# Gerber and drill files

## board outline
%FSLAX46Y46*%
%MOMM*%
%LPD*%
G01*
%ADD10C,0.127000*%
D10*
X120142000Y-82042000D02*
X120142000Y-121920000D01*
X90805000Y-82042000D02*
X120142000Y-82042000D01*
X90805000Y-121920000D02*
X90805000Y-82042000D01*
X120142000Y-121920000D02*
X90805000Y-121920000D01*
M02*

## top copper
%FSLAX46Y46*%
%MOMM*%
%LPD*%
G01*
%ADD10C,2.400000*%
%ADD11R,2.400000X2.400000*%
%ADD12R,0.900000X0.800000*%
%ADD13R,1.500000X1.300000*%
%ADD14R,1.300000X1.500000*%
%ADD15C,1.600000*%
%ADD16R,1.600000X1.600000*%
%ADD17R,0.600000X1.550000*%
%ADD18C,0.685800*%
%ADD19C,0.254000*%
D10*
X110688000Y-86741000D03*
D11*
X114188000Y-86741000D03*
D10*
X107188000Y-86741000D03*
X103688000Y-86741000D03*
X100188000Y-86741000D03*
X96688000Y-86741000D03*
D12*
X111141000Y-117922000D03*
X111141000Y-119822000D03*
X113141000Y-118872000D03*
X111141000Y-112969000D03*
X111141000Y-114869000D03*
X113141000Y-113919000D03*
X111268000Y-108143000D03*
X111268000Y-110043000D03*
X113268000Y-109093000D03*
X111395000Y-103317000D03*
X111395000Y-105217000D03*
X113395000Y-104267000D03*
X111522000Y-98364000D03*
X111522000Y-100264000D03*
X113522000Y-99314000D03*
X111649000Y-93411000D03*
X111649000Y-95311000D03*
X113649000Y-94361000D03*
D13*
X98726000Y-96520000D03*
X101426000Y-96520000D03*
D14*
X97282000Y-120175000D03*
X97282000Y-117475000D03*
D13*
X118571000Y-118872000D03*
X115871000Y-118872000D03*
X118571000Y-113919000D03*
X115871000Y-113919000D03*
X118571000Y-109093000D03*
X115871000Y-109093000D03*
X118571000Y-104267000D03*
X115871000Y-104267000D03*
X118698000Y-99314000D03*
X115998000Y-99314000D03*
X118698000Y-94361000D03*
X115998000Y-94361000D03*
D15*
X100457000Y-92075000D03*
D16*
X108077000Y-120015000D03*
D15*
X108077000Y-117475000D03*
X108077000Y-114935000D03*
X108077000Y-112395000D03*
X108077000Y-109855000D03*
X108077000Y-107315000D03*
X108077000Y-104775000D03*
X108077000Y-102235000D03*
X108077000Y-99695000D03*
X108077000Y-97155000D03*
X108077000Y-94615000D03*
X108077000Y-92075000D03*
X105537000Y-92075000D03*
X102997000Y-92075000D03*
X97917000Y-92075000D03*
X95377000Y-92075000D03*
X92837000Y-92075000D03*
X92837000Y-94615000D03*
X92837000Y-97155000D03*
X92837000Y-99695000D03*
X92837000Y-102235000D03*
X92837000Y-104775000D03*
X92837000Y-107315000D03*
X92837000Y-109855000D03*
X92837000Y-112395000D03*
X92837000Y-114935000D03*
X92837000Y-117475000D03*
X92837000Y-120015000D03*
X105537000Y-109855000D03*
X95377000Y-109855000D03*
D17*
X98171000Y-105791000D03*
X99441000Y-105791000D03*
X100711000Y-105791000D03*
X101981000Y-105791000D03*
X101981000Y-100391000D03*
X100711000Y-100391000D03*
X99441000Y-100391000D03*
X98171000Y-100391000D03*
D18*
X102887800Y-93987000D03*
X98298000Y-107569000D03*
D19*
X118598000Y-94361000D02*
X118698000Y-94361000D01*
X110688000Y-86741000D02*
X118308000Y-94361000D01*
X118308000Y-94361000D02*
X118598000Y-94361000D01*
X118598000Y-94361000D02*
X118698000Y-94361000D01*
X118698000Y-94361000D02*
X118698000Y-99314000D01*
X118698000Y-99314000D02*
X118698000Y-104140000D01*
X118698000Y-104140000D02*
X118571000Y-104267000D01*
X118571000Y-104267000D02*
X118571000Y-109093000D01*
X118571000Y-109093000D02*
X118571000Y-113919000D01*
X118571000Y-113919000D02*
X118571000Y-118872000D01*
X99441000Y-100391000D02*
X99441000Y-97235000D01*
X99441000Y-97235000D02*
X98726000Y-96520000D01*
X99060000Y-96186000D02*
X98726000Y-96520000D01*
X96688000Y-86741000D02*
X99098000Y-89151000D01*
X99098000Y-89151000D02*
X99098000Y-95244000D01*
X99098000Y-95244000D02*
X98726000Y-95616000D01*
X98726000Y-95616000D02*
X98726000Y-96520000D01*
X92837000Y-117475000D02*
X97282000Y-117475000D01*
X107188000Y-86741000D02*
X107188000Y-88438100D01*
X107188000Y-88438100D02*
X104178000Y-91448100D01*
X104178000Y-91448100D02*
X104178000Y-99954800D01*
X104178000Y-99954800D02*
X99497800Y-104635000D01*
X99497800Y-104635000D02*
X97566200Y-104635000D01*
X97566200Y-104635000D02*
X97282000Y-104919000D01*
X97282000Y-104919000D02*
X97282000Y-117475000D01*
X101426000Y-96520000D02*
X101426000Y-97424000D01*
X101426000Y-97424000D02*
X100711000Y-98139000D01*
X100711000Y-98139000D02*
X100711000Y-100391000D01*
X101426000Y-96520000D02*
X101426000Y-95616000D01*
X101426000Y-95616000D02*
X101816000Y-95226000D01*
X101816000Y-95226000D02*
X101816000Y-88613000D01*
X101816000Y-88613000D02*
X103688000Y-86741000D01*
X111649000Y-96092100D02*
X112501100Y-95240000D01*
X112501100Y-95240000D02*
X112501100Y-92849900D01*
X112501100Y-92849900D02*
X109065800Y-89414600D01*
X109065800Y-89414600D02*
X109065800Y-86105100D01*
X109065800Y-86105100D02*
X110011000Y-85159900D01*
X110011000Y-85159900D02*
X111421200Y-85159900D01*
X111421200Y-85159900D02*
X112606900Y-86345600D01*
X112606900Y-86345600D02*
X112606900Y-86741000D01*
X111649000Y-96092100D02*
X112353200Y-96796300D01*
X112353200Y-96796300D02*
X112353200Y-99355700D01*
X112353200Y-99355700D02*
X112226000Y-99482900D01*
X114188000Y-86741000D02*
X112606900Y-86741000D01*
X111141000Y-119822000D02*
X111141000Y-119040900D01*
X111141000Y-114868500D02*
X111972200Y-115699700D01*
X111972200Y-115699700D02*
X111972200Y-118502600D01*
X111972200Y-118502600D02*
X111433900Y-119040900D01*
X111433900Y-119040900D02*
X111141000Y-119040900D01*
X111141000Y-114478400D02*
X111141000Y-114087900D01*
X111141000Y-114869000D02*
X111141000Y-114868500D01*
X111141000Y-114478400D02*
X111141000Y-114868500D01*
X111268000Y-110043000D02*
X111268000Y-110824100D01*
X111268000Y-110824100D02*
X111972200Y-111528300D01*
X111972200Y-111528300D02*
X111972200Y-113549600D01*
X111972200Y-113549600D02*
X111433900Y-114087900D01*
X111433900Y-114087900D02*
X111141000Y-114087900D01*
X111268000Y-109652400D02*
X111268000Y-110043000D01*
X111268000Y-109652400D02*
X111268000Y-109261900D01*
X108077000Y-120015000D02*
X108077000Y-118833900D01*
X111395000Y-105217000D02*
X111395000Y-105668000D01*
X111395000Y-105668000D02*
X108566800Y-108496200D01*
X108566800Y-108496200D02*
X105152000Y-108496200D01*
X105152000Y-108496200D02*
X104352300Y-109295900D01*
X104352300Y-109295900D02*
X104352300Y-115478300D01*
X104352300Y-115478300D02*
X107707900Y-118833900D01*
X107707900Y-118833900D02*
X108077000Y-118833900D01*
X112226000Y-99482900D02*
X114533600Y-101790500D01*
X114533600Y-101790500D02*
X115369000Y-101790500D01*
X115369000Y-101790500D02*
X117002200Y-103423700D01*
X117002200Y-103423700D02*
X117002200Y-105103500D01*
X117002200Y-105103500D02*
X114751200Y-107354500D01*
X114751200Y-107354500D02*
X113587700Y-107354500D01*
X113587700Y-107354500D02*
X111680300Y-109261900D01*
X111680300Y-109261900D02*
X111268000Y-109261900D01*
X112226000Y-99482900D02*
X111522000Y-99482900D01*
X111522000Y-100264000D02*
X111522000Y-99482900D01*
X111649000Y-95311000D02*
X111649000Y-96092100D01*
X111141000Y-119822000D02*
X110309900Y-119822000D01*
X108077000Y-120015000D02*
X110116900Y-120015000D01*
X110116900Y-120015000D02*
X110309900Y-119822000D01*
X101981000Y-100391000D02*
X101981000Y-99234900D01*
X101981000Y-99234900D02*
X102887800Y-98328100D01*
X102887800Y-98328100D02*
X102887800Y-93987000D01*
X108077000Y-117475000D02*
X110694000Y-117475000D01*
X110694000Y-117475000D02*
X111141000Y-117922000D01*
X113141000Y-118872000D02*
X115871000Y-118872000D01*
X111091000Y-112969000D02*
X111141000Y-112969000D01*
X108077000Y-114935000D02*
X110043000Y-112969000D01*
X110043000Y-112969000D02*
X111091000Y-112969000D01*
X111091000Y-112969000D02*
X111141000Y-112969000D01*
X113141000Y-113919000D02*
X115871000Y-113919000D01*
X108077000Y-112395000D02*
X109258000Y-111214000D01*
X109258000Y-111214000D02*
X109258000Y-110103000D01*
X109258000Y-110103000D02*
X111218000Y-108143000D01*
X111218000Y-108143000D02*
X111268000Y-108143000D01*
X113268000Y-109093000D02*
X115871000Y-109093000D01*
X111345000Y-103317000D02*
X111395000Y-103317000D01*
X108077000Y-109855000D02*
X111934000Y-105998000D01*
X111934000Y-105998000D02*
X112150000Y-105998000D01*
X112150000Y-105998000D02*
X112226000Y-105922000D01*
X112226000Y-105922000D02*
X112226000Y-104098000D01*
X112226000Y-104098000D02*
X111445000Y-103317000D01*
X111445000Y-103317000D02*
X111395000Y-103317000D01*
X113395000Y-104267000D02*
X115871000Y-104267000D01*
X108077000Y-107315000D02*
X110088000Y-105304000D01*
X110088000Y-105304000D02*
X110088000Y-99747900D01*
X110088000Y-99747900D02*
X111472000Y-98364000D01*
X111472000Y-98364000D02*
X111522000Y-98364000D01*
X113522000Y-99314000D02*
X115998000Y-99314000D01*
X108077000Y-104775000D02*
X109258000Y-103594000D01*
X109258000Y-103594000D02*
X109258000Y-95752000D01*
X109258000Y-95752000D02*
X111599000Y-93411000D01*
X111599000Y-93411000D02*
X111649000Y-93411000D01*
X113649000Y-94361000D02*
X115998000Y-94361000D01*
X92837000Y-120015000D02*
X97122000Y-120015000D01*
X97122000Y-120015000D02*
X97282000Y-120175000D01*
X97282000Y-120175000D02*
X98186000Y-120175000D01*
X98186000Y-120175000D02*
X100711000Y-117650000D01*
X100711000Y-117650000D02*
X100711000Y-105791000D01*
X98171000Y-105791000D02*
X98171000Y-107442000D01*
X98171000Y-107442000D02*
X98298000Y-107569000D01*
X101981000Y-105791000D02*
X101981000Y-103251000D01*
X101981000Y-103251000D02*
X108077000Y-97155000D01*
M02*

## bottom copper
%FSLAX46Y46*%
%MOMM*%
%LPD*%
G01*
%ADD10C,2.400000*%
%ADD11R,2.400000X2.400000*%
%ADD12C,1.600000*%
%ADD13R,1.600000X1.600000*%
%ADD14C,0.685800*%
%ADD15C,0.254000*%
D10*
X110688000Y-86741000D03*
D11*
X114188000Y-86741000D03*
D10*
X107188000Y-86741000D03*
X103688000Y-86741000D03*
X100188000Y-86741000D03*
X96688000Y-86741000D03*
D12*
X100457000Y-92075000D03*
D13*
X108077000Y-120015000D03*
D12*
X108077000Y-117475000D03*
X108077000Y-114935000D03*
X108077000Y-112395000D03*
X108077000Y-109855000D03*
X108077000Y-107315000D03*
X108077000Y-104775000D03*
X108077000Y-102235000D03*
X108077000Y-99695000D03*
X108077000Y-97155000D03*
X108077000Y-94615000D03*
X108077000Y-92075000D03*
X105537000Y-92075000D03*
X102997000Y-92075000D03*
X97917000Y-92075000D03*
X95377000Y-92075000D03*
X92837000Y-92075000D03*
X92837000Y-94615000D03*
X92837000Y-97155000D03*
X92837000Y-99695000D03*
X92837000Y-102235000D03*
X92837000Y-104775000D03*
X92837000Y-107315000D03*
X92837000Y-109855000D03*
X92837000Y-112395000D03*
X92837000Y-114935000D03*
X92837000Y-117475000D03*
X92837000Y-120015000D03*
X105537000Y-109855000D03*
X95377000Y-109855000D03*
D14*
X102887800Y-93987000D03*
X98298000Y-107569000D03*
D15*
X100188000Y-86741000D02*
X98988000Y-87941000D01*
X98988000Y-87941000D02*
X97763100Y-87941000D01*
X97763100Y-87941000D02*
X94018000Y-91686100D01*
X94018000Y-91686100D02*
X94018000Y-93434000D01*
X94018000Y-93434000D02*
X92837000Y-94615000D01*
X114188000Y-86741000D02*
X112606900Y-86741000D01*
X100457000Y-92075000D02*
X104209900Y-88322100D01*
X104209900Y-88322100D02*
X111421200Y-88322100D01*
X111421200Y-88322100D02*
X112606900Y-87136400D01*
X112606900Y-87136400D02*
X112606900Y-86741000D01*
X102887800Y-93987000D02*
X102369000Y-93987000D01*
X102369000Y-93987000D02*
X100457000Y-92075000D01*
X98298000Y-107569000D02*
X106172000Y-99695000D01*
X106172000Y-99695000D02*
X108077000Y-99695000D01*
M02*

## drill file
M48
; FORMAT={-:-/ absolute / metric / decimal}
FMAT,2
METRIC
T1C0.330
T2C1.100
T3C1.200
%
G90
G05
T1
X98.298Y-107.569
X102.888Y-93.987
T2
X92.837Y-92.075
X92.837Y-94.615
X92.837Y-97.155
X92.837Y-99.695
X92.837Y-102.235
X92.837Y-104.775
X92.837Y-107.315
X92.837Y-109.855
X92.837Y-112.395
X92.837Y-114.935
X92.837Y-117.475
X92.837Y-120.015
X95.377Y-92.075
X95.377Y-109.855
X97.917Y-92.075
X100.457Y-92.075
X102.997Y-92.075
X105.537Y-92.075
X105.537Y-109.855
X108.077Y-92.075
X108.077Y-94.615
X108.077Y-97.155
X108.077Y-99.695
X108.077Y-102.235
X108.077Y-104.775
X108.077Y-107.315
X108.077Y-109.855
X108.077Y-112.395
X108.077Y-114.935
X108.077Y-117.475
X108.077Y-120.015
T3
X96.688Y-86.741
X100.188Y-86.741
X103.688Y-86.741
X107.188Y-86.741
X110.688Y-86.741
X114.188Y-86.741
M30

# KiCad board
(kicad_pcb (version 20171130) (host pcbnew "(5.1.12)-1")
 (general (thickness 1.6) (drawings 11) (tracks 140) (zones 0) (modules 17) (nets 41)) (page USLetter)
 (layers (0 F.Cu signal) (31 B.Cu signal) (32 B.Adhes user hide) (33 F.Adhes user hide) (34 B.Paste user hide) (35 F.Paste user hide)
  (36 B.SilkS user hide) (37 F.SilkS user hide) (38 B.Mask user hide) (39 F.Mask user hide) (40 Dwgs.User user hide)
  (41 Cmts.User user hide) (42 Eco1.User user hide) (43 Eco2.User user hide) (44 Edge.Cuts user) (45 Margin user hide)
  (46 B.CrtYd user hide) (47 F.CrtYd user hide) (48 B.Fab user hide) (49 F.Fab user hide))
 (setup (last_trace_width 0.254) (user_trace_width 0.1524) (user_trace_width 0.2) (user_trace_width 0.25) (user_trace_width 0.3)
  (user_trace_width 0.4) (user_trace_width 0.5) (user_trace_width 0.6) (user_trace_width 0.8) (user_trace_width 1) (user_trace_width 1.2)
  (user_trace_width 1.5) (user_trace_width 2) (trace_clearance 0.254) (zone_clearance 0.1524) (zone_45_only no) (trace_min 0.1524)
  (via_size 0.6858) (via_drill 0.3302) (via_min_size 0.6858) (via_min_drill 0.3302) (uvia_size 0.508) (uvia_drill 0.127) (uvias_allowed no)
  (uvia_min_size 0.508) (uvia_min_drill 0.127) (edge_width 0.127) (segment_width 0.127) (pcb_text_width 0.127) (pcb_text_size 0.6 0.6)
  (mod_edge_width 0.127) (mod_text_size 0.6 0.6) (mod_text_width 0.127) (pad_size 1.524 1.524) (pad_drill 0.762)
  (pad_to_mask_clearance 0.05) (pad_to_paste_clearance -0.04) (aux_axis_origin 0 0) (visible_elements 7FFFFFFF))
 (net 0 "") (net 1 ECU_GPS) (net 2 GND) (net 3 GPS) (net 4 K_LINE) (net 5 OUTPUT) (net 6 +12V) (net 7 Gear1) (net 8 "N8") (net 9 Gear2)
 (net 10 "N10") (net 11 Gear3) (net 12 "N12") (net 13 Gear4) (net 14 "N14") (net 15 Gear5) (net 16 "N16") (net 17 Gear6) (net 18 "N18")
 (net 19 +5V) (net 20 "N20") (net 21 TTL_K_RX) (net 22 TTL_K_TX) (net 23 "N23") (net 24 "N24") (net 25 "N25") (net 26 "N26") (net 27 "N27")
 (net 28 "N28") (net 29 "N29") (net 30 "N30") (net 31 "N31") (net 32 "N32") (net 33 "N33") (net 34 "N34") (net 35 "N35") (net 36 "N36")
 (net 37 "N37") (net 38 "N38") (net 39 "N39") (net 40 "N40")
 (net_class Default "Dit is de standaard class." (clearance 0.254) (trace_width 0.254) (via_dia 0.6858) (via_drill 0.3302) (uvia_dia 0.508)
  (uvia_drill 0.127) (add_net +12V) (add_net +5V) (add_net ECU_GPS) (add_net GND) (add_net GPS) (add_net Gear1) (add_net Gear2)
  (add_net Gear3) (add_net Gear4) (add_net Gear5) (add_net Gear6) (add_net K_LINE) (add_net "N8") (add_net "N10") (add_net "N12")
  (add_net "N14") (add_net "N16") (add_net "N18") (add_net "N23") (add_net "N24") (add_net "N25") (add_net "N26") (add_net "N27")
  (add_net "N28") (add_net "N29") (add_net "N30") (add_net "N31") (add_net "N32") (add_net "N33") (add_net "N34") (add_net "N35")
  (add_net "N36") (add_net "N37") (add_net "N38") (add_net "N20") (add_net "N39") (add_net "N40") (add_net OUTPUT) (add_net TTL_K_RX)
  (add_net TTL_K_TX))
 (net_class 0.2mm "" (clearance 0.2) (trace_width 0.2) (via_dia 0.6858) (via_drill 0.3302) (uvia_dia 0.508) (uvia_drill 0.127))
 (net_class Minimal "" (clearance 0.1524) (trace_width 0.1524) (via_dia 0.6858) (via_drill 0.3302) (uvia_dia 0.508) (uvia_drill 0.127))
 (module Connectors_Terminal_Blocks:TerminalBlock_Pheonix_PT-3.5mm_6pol (layer F.Cu) (at 114.188 86.741 180)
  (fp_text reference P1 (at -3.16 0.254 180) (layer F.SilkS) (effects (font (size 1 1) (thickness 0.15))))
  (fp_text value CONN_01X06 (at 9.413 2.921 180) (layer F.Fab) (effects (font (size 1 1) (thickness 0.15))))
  (pad 2 thru_hole circle (at 3.5 0 180) (size 2.4 2.4) (drill 1.2) (layers *.Cu *.Mask) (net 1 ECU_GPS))
  (pad 1 thru_hole rect (at 0 0 180) (size 2.4 2.4) (drill 1.2) (layers *.Cu *.Mask) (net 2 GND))
  (pad 3 thru_hole circle (at 7 0 180) (size 2.4 2.4) (drill 1.2) (layers *.Cu *.Mask) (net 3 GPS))
  (pad 4 thru_hole circle (at 10.5 0 180) (size 2.4 2.4) (drill 1.2) (layers *.Cu *.Mask) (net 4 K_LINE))
  (pad 5 thru_hole circle (at 14 0 180) (size 2.4 2.4) (drill 1.2) (layers *.Cu *.Mask) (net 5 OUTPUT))
  (pad 6 thru_hole circle (at 17.5 0 180) (size 2.4 2.4) (drill 1.2) (layers *.Cu *.Mask) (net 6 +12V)))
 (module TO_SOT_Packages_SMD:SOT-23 (layer F.Cu) (at 112.141 118.872)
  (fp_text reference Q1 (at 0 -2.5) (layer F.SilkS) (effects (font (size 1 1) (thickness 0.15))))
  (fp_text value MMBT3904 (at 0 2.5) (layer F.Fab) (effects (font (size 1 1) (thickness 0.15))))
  (pad 1 smd rect (at -1 -0.95) (size 0.9 0.8) (layers F.Cu F.Paste F.Mask) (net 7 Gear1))
  (pad 2 smd rect (at -1 0.95) (size 0.9 0.8) (layers F.Cu F.Paste F.Mask) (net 2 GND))
  (pad 3 smd rect (at 1 0) (size 0.9 0.8) (layers F.Cu F.Paste F.Mask) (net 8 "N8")))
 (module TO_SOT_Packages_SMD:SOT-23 (layer F.Cu) (at 112.141 113.919)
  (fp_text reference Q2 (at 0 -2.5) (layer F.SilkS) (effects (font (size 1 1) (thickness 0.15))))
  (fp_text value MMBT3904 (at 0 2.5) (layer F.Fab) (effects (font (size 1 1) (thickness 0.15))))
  (pad 1 smd rect (at -1 -0.95) (size 0.9 0.8) (layers F.Cu F.Paste F.Mask) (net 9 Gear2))
  (pad 2 smd rect (at -1 0.95) (size 0.9 0.8) (layers F.Cu F.Paste F.Mask) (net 2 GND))
  (pad 3 smd rect (at 1 0) (size 0.9 0.8) (layers F.Cu F.Paste F.Mask) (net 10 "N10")))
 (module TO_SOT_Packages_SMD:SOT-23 (layer F.Cu) (at 112.268 109.093)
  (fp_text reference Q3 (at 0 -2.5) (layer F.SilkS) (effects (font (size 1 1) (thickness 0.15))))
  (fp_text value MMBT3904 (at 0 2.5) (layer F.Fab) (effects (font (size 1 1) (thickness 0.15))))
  (pad 1 smd rect (at -1 -0.95) (size 0.9 0.8) (layers F.Cu F.Paste F.Mask) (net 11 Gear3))
  (pad 2 smd rect (at -1 0.95) (size 0.9 0.8) (layers F.Cu F.Paste F.Mask) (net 2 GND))
  (pad 3 smd rect (at 1 0) (size 0.9 0.8) (layers F.Cu F.Paste F.Mask) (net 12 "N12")))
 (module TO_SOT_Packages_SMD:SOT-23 (layer F.Cu) (at 112.395 104.267)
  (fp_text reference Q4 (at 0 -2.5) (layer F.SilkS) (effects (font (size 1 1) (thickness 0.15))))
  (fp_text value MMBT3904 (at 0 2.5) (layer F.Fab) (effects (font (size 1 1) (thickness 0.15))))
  (pad 1 smd rect (at -1 -0.95) (size 0.9 0.8) (layers F.Cu F.Paste F.Mask) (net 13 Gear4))
  (pad 2 smd rect (at -1 0.95) (size 0.9 0.8) (layers F.Cu F.Paste F.Mask) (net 2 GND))
  (pad 3 smd rect (at 1 0) (size 0.9 0.8) (layers F.Cu F.Paste F.Mask) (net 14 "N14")))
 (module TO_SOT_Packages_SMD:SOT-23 (layer F.Cu) (at 112.522 99.314)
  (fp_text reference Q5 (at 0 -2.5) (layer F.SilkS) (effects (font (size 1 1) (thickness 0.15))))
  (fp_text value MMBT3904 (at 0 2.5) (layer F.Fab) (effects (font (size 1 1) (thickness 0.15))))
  (pad 1 smd rect (at -1 -0.95) (size 0.9 0.8) (layers F.Cu F.Paste F.Mask) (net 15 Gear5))
  (pad 2 smd rect (at -1 0.95) (size 0.9 0.8) (layers F.Cu F.Paste F.Mask) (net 2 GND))
  (pad 3 smd rect (at 1 0) (size 0.9 0.8) (layers F.Cu F.Paste F.Mask) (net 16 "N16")))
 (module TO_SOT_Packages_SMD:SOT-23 (layer F.Cu) (at 112.649 94.361)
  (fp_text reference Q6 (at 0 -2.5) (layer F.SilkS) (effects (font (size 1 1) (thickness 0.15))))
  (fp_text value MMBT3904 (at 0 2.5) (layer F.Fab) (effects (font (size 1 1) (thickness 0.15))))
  (pad 1 smd rect (at -1 -0.95) (size 0.9 0.8) (layers F.Cu F.Paste F.Mask) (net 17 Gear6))
  (pad 2 smd rect (at -1 0.95) (size 0.9 0.8) (layers F.Cu F.Paste F.Mask) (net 2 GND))
  (pad 3 smd rect (at 1 0) (size 0.9 0.8) (layers F.Cu F.Paste F.Mask) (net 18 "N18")))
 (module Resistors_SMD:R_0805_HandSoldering (layer F.Cu) (at 100.076 96.52)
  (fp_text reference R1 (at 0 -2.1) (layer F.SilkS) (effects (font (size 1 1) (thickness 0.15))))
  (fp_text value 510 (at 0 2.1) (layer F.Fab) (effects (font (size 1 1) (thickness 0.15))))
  (pad 1 smd rect (at -1.35 0) (size 1.5 1.3) (layers F.Cu F.Paste F.Mask) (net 6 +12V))
  (pad 2 smd rect (at 1.35 0) (size 1.5 1.3) (layers F.Cu F.Paste F.Mask) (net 4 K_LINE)))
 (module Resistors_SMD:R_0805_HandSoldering (layer F.Cu) (at 97.282 118.825 90)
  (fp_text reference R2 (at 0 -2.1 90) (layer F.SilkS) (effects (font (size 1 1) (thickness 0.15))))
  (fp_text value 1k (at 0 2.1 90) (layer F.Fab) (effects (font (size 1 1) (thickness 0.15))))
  (pad 1 smd rect (at -1.35 0 90) (size 1.5 1.3) (layers F.Cu F.Paste F.Mask) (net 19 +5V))
  (pad 2 smd rect (at 1.35 0 90) (size 1.5 1.3) (layers F.Cu F.Paste F.Mask) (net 3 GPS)))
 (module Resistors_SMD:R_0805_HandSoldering (layer F.Cu) (at 117.221 118.872 180)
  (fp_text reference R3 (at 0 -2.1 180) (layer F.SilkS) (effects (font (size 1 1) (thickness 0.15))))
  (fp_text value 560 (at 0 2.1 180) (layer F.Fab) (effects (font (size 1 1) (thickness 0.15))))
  (pad 1 smd rect (at -1.35 0 180) (size 1.5 1.3) (layers F.Cu F.Paste F.Mask) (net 1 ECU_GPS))
  (pad 2 smd rect (at 1.35 0 180) (size 1.5 1.3) (layers F.Cu F.Paste F.Mask) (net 8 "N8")))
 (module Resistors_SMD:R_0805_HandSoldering (layer F.Cu) (at 117.221 113.919 180)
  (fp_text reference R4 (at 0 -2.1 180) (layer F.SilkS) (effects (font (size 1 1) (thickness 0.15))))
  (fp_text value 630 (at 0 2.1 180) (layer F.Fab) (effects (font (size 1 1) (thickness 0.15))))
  (pad 1 smd rect (at -1.35 0 180) (size 1.5 1.3) (layers F.Cu F.Paste F.Mask) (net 1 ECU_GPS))
  (pad 2 smd rect (at 1.35 0 180) (size 1.5 1.3) (layers F.Cu F.Paste F.Mask) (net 10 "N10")))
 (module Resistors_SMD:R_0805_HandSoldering (layer F.Cu) (at 117.221 109.093 180)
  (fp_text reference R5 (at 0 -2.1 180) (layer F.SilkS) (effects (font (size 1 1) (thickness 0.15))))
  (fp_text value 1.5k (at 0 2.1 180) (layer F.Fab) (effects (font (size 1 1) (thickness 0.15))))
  (pad 1 smd rect (at -1.35 0 180) (size 1.5 1.3) (layers F.Cu F.Paste F.Mask) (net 1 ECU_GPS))
  (pad 2 smd rect (at 1.35 0 180) (size 1.5 1.3) (layers F.Cu F.Paste F.Mask) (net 12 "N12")))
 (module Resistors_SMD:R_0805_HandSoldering (layer F.Cu) (at 117.221 104.267 180)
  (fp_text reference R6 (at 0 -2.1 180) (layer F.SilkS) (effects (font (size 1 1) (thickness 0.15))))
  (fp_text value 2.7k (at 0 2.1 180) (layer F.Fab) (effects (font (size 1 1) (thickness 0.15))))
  (pad 1 smd rect (at -1.35 0 180) (size 1.5 1.3) (layers F.Cu F.Paste F.Mask) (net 1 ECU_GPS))
  (pad 2 smd rect (at 1.35 0 180) (size 1.5 1.3) (layers F.Cu F.Paste F.Mask) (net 14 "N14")))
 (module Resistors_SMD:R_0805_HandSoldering (layer F.Cu) (at 117.348 99.314 180)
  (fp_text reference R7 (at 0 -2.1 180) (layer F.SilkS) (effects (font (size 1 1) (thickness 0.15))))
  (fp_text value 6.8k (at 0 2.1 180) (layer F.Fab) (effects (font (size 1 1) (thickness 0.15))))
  (pad 1 smd rect (at -1.35 0 180) (size 1.5 1.3) (layers F.Cu F.Paste F.Mask) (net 1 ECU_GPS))
  (pad 2 smd rect (at 1.35 0 180) (size 1.5 1.3) (layers F.Cu F.Paste F.Mask) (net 16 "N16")))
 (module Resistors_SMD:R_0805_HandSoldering (layer F.Cu) (at 117.348 94.361 180)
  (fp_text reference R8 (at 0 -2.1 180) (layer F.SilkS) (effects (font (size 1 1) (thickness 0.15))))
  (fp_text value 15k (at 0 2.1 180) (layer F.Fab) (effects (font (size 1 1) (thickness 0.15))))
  (pad 1 smd rect (at -1.35 0 180) (size 1.5 1.3) (layers F.Cu F.Paste F.Mask) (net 1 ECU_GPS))
  (pad 2 smd rect (at 1.35 0 180) (size 1.5 1.3) (layers F.Cu F.Paste F.Mask) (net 18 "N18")))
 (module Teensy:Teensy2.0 (layer F.Cu) (at 100.457 106.045 90)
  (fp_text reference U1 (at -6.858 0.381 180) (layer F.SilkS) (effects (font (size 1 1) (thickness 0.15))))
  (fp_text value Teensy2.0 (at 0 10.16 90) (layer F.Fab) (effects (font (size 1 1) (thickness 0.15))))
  (pad 15 thru_hole circle (at 13.97 0 90) (size 1.6 1.6) (drill 1.1) (layers *.Cu *.Mask F.SilkS) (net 2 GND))
  (pad 1 thru_hole rect (at -13.97 7.62 90) (size 1.6 1.6) (drill 1.1) (layers *.Cu *.Mask F.SilkS) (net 2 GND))
  (pad 2 thru_hole circle (at -11.43 7.62 90) (size 1.6 1.6) (drill 1.1) (layers *.Cu *.Mask F.SilkS) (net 7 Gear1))
  (pad 3 thru_hole circle (at -8.89 7.62 90) (size 1.6 1.6) (drill 1.1) (layers *.Cu *.Mask F.SilkS) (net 9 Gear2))
  (pad 4 thru_hole circle (at -6.35 7.62 90) (size 1.6 1.6) (drill 1.1) (layers *.Cu *.Mask F.SilkS) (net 11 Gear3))
  (pad 5 thru_hole circle (at -3.81 7.62 90) (size 1.6 1.6) (drill 1.1) (layers *.Cu *.Mask F.SilkS) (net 13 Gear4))
  (pad 6 thru_hole circle (at -1.27 7.62 90) (size 1.6 1.6) (drill 1.1) (layers *.Cu *.Mask F.SilkS) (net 15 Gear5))
  (pad 7 thru_hole circle (at 1.27 7.62 90) (size 1.6 1.6) (drill 1.1) (layers *.Cu *.Mask F.SilkS) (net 17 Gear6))
  (pad 8 thru_hole circle (at 3.81 7.62 90) (size 1.6 1.6) (drill 1.1) (layers *.Cu *.Mask F.SilkS) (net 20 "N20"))
  (pad 9 thru_hole circle (at 6.35 7.62 90) (size 1.6 1.6) (drill 1.1) (layers *.Cu *.Mask F.SilkS) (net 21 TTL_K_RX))
  (pad 10 thru_hole circle (at 8.89 7.62 90) (size 1.6 1.6) (drill 1.1) (layers *.Cu *.Mask F.SilkS) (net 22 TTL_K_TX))
  (pad 11 thru_hole circle (at 11.43 7.62 90) (size 1.6 1.6) (drill 1.1) (layers *.Cu *.Mask F.SilkS) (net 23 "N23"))
  (pad 12 thru_hole circle (at 13.97 7.62 90) (size 1.6 1.6) (drill 1.1) (layers *.Cu *.Mask F.SilkS) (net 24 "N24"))
  (pad 13 thru_hole circle (at 13.97 5.08 90) (size 1.6 1.6) (drill 1.1) (layers *.Cu *.Mask F.SilkS) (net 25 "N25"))
  (pad 14 thru_hole circle (at 13.97 2.54 90) (size 1.6 1.6) (drill 1.1) (layers *.Cu *.Mask F.SilkS) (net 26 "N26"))
  (pad 16 thru_hole circle (at 13.97 -2.54 90) (size 1.6 1.6) (drill 1.1) (layers *.Cu *.Mask F.SilkS) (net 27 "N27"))
  (pad 17 thru_hole circle (at 13.97 -5.08 90) (size 1.6 1.6) (drill 1.1) (layers *.Cu *.Mask F.SilkS) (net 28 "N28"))
  (pad 18 thru_hole circle (at 13.97 -7.62 90) (size 1.6 1.6) (drill 1.1) (layers *.Cu *.Mask F.SilkS) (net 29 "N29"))
  (pad 19 thru_hole circle (at 11.43 -7.62 90) (size 1.6 1.6) (drill 1.1) (layers *.Cu *.Mask F.SilkS) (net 5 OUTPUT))
  (pad 20 thru_hole circle (at 8.89 -7.62 90) (size 1.6 1.6) (drill 1.1) (layers *.Cu *.Mask F.SilkS) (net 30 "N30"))
  (pad 21 thru_hole circle (at 6.35 -7.62 90) (size 1.6 1.6) (drill 1.1) (layers *.Cu *.Mask F.SilkS) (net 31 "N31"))
  (pad 22 thru_hole circle (at 3.81 -7.62 90) (size 1.6 1.6) (drill 1.1) (layers *.Cu *.Mask F.SilkS) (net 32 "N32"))
  (pad 23 thru_hole circle (at 1.27 -7.62 90) (size 1.6 1.6) (drill 1.1) (layers *.Cu *.Mask F.SilkS) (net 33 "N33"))
  (pad 24 thru_hole circle (at -1.27 -7.62 90) (size 1.6 1.6) (drill 1.1) (layers *.Cu *.Mask F.SilkS) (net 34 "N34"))
  (pad 25 thru_hole circle (at -3.81 -7.62 90) (size 1.6 1.6) (drill 1.1) (layers *.Cu *.Mask F.SilkS) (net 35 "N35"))
  (pad 26 thru_hole circle (at -6.35 -7.62 90) (size 1.6 1.6) (drill 1.1) (layers *.Cu *.Mask F.SilkS))
  (pad 27 thru_hole circle (at -8.89 -7.62 90) (size 1.6 1.6) (drill 1.1) (layers *.Cu *.Mask F.SilkS) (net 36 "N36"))
  (pad 28 thru_hole circle (at -11.43 -7.62 90) (size 1.6 1.6) (drill 1.1) (layers *.Cu *.Mask F.SilkS) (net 3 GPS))
  (pad 29 thru_hole circle (at -13.97 -7.62 90) (size 1.6 1.6) (drill 1.1) (layers *.Cu *.Mask F.SilkS) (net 19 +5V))
  (pad 30 thru_hole circle (at -3.81 5.08 90) (size 1.6 1.6) (drill 1.1) (layers *.Cu *.Mask F.SilkS) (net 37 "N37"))
  (pad 31 thru_hole circle (at -3.81 -5.08 90) (size 1.6 1.6) (drill 1.1) (layers *.Cu *.Mask F.SilkS) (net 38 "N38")))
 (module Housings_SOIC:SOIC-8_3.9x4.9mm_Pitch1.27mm (layer F.Cu) (at 100.076 103.091 90)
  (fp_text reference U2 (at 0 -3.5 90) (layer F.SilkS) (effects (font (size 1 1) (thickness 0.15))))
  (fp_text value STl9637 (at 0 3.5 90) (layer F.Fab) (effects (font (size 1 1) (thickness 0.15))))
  (pad 1 smd rect (at -2.7 -1.905 90) (size 1.55 0.6) (layers F.Cu F.Paste F.Mask) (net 21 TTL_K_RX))
  (pad 2 smd rect (at -2.7 -0.635 90) (size 1.55 0.6) (layers F.Cu F.Paste F.Mask) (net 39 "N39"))
  (pad 3 smd rect (at -2.7 0.635 90) (size 1.55 0.6) (layers F.Cu F.Paste F.Mask) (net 19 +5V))
  (pad 4 smd rect (at -2.7 1.905 90) (size 1.55 0.6) (layers F.Cu F.Paste F.Mask) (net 22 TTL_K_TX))
  (pad 5 smd rect (at 2.7 1.905 90) (size 1.55 0.6) (layers F.Cu F.Paste F.Mask) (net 2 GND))
  (pad 6 smd rect (at 2.7 0.635 90) (size 1.55 0.6) (layers F.Cu F.Paste F.Mask) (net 4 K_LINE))
  (pad 7 smd rect (at 2.7 -0.635 90) (size 1.55 0.6) (layers F.Cu F.Paste F.Mask) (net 6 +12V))
  (pad 8 smd rect (at 2.7 -1.905 90) (size 1.55 0.6) (layers F.Cu F.Paste F.Mask) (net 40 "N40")))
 (gr_line (start 120.142 82.042) (end 120.142 121.92) (layer Edge.Cuts) (width 0.127))
 (gr_line (start 90.805 82.042) (end 120.142 82.042) (layer Edge.Cuts) (width 0.127))
 (gr_line (start 90.805 121.92) (end 90.805 82.042) (layer Edge.Cuts) (width 0.127))
 (gr_line (start 120.142 121.92) (end 90.805 121.92) (layer Edge.Cuts) (width 0.127))
 (segment (start 118.598 94.361) (end 118.698 94.361) (width 0.254) (layer F.Cu) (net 1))
 (segment (start 110.688 86.741) (end 118.308 94.361) (width 0.254) (layer F.Cu) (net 1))
 (segment (start 118.308 94.361) (end 118.598 94.361) (width 0.254) (layer F.Cu) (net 1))
 (segment (start 118.598 94.361) (end 118.698 94.361) (width 0.254) (layer F.Cu) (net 1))
 (segment (start 118.698 94.361) (end 118.698 99.314) (width 0.254) (layer F.Cu) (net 1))
 (segment (start 118.698 99.314) (end 118.698 104.14) (width 0.254) (layer F.Cu) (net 1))
 (segment (start 118.698 104.14) (end 118.571 104.267) (width 0.254) (layer F.Cu) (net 1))
 (segment (start 118.571 104.267) (end 118.571 109.093) (width 0.254) (layer F.Cu) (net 1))
 (segment (start 118.571 109.093) (end 118.571 113.919) (width 0.254) (layer F.Cu) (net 1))
 (segment (start 118.571 113.919) (end 118.571 118.872) (width 0.254) (layer F.Cu) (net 1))
 (segment (start 99.441 100.391) (end 99.441 97.235) (width 0.254) (layer F.Cu) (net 6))
 (segment (start 99.441 97.235) (end 98.726 96.52) (width 0.254) (layer F.Cu) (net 6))
 (segment (start 99.06 96.186) (end 98.726 96.52) (width 0.254) (layer F.Cu) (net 6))
 (segment (start 96.688 86.741) (end 99.098 89.151) (width 0.254) (layer F.Cu) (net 6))
 (segment (start 99.098 89.151) (end 99.098 95.244) (width 0.254) (layer F.Cu) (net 6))
 (segment (start 99.098 95.244) (end 98.726 95.616) (width 0.254) (layer F.Cu) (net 6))
 (segment (start 98.726 95.616) (end 98.726 96.52) (width 0.254) (layer F.Cu) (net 6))
 (segment (start 92.837 117.475) (end 97.282 117.475) (width 0.254) (layer F.Cu) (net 3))
 (segment (start 107.188 86.741) (end 107.188 88.4381) (width 0.254) (layer F.Cu) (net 3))
 (segment (start 107.188 88.4381) (end 104.178 91.4481) (width 0.254) (layer F.Cu) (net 3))
 (segment (start 104.178 91.4481) (end 104.178 99.9548) (width 0.254) (layer F.Cu) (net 3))
 (segment (start 104.178 99.9548) (end 99.4978 104.635) (width 0.254) (layer F.Cu) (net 3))
 (segment (start 99.4978 104.635) (end 97.5662 104.635) (width 0.254) (layer F.Cu) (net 3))
 (segment (start 97.5662 104.635) (end 97.282 104.919) (width 0.254) (layer F.Cu) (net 3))
 (segment (start 97.282 104.919) (end 97.282 117.475) (width 0.254) (layer F.Cu) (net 3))
 (segment (start 101.426 96.52) (end 101.426 97.424) (width 0.254) (layer F.Cu) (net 4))
 (segment (start 101.426 97.424) (end 100.711 98.139) (width 0.254) (layer F.Cu) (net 4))
 (segment (start 100.711 98.139) (end 100.711 100.391) (width 0.254) (layer F.Cu) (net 4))
 (segment (start 101.426 96.52) (end 101.426 95.616) (width 0.254) (layer F.Cu) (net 4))
 (segment (start 101.426 95.616) (end 101.816 95.226) (width 0.254) (layer F.Cu) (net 4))
 (segment (start 101.816 95.226) (end 101.816 88.613) (width 0.254) (layer F.Cu) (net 4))
 (segment (start 101.816 88.613) (end 103.688 86.741) (width 0.254) (layer F.Cu) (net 4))
 (segment (start 100.188 86.741) (end 98.988 87.941) (width 0.254) (layer B.Cu) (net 5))
 (segment (start 98.988 87.941) (end 97.7631 87.941) (width 0.254) (layer B.Cu) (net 5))
 (segment (start 97.7631 87.941) (end 94.018 91.6861) (width 0.254) (layer B.Cu) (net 5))
 (segment (start 94.018 91.6861) (end 94.018 93.434) (width 0.254) (layer B.Cu) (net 5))
 (segment (start 94.018 93.434) (end 92.837 94.615) (width 0.254) (layer B.Cu) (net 5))
 (segment (start 111.649 96.0921) (end 112.5011 95.24) (width 0.254) (layer F.Cu) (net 2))
 (segment (start 112.5011 95.24) (end 112.5011 92.8499) (width 0.254) (layer F.Cu) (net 2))
 (segment (start 112.5011 92.8499) (end 109.0658 89.4146) (width 0.254) (layer F.Cu) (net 2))
 (segment (start 109.0658 89.4146) (end 109.0658 86.1051) (width 0.254) (layer F.Cu) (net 2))
 (segment (start 109.0658 86.1051) (end 110.011 85.1599) (width 0.254) (layer F.Cu) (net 2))
 (segment (start 110.011 85.1599) (end 111.4212 85.1599) (width 0.254) (layer F.Cu) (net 2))
 (segment (start 111.4212 85.1599) (end 112.6069 86.3456) (width 0.254) (layer F.Cu) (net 2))
 (segment (start 112.6069 86.3456) (end 112.6069 86.741) (width 0.254) (layer F.Cu) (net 2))
 (segment (start 111.649 96.0921) (end 112.3532 96.7963) (width 0.254) (layer F.Cu) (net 2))
 (segment (start 112.3532 96.7963) (end 112.3532 99.3557) (width 0.254) (layer F.Cu) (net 2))
 (segment (start 112.3532 99.3557) (end 112.226 99.4829) (width 0.254) (layer F.Cu) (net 2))
 (segment (start 114.188 86.741) (end 112.6069 86.741) (width 0.254) (layer F.Cu) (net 2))
 (segment (start 111.141 119.822) (end 111.141 119.0409) (width 0.254) (layer F.Cu) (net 2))
 (segment (start 111.141 114.8685) (end 111.9722 115.6997) (width 0.254) (layer F.Cu) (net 2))
 (segment (start 111.9722 115.6997) (end 111.9722 118.5026) (width 0.254) (layer F.Cu) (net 2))
 (segment (start 111.9722 118.5026) (end 111.4339 119.0409) (width 0.254) (layer F.Cu) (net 2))
 (segment (start 111.4339 119.0409) (end 111.141 119.0409) (width 0.254) (layer F.Cu) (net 2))
 (segment (start 111.141 114.4784) (end 111.141 114.0879) (width 0.254) (layer F.Cu) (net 2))
 (segment (start 111.141 114.869) (end 111.141 114.8685) (width 0.254) (layer F.Cu) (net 2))
 (segment (start 111.141 114.4784) (end 111.141 114.8685) (width 0.254) (layer F.Cu) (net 2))
 (segment (start 111.268 110.043) (end 111.268 110.8241) (width 0.254) (layer F.Cu) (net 2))
 (segment (start 111.268 110.8241) (end 111.9722 111.5283) (width 0.254) (layer F.Cu) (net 2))
 (segment (start 111.9722 111.5283) (end 111.9722 113.5496) (width 0.254) (layer F.Cu) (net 2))
 (segment (start 111.9722 113.5496) (end 111.4339 114.0879) (width 0.254) (layer F.Cu) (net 2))
 (segment (start 111.4339 114.0879) (end 111.141 114.0879) (width 0.254) (layer F.Cu) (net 2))
 (segment (start 111.268 109.6524) (end 111.268 110.043) (width 0.254) (layer F.Cu) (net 2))
 (segment (start 111.268 109.6524) (end 111.268 109.2619) (width 0.254) (layer F.Cu) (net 2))
 (segment (start 108.077 120.015) (end 108.077 118.8339) (width 0.254) (layer F.Cu) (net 2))
 (segment (start 111.395 105.217) (end 111.395 105.668) (width 0.254) (layer F.Cu) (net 2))
 (segment (start 111.395 105.668) (end 108.5668 108.4962) (width 0.254) (layer F.Cu) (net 2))
 (segment (start 108.5668 108.4962) (end 105.152 108.4962) (width 0.254) (layer F.Cu) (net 2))
 (segment (start 105.152 108.4962) (end 104.3523 109.2959) (width 0.254) (layer F.Cu) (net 2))
 (segment (start 104.3523 109.2959) (end 104.3523 115.4783) (width 0.254) (layer F.Cu) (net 2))
 (segment (start 104.3523 115.4783) (end 107.7079 118.8339) (width 0.254) (layer F.Cu) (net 2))
 (segment (start 107.7079 118.8339) (end 108.077 118.8339) (width 0.254) (layer F.Cu) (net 2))
 (segment (start 112.226 99.4829) (end 114.5336 101.7905) (width 0.254) (layer F.Cu) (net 2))
 (segment (start 114.5336 101.7905) (end 115.369 101.7905) (width 0.254) (layer F.Cu) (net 2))
 (segment (start 115.369 101.7905) (end 117.0022 103.4237) (width 0.254) (layer F.Cu) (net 2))
 (segment (start 117.0022 103.4237) (end 117.0022 105.1035) (width 0.254) (layer F.Cu) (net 2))
 (segment (start 117.0022 105.1035) (end 114.7512 107.3545) (width 0.254) (layer F.Cu) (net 2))
 (segment (start 114.7512 107.3545) (end 113.5877 107.3545) (width 0.254) (layer F.Cu) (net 2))
 (segment (start 113.5877 107.3545) (end 111.6803 109.2619) (width 0.254) (layer F.Cu) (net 2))
 (segment (start 111.6803 109.2619) (end 111.268 109.2619) (width 0.254) (layer F.Cu) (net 2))
 (segment (start 112.226 99.4829) (end 111.522 99.4829) (width 0.254) (layer F.Cu) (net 2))
 (segment (start 111.522 100.264) (end 111.522 99.4829) (width 0.254) (layer F.Cu) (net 2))
 (segment (start 111.649 95.311) (end 111.649 96.0921) (width 0.254) (layer F.Cu) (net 2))
 (segment (start 114.188 86.741) (end 112.6069 86.741) (width 0.254) (layer B.Cu) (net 2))
 (segment (start 100.457 92.075) (end 104.2099 88.3221) (width 0.254) (layer B.Cu) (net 2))
 (segment (start 104.2099 88.3221) (end 111.4212 88.3221) (width 0.254) (layer B.Cu) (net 2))
 (segment (start 111.4212 88.3221) (end 112.6069 87.1364) (width 0.254) (layer B.Cu) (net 2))
 (segment (start 112.6069 87.1364) (end 112.6069 86.741) (width 0.254) (layer B.Cu) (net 2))
 (segment (start 111.141 119.822) (end 110.3099 119.822) (width 0.254) (layer F.Cu) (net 2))
 (segment (start 108.077 120.015) (end 110.1169 120.015) (width 0.254) (layer F.Cu) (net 2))
 (segment (start 110.1169 120.015) (end 110.3099 119.822) (width 0.254) (layer F.Cu) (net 2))
 (segment (start 101.981 100.391) (end 101.981 99.2349) (width 0.254) (layer F.Cu) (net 2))
 (segment (start 102.8878 93.987) (end 102.369 93.987) (width 0.254) (layer B.Cu) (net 2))
 (segment (start 102.369 93.987) (end 100.457 92.075) (width 0.254) (layer B.Cu) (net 2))
 (segment (start 101.981 99.2349) (end 102.8878 98.3281) (width 0.254) (layer F.Cu) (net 2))
 (segment (start 102.8878 98.3281) (end 102.8878 93.987) (width 0.254) (layer F.Cu) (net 2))
 (via (at 102.8878 93.987) (size 0.6858) (layers F.Cu B.Cu) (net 2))
 (segment (start 108.077 117.475) (end 110.694 117.475) (width 0.254) (layer F.Cu) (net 7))
 (segment (start 110.694 117.475) (end 111.141 117.922) (width 0.254) (layer F.Cu) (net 7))
 (segment (start 113.141 118.872) (end 115.871 118.872) (width 0.254) (layer F.Cu) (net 8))
 (segment (start 111.091 112.969) (end 111.141 112.969) (width 0.254) (layer F.Cu) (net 9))
 (segment (start 108.077 114.935) (end 110.043 112.969) (width 0.254) (layer F.Cu) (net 9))
 (segment (start 110.043 112.969) (end 111.091 112.969) (width 0.254) (layer F.Cu) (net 9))
 (segment (start 111.091 112.969) (end 111.141 112.969) (width 0.254) (layer F.Cu) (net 9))
 (segment (start 113.141 113.919) (end 115.871 113.919) (width 0.254) (layer F.Cu) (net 10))
 (segment (start 108.077 112.395) (end 109.258 111.214) (width 0.254) (layer F.Cu) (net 11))
 (segment (start 109.258 111.214) (end 109.258 110.103) (width 0.254) (layer F.Cu) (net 11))
 (segment (start 109.258 110.103) (end 111.218 108.143) (width 0.254) (layer F.Cu) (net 11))
 (segment (start 111.218 108.143) (end 111.268 108.143) (width 0.254) (layer F.Cu) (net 11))
 (segment (start 113.268 109.093) (end 115.871 109.093) (width 0.254) (layer F.Cu) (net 12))
 (segment (start 111.345 103.317) (end 111.395 103.317) (width 0.254) (layer F.Cu) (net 13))
 (segment (start 108.077 109.855) (end 111.934 105.998) (width 0.254) (layer F.Cu) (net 13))
 (segment (start 111.934 105.998) (end 112.15 105.998) (width 0.254) (layer F.Cu) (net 13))
 (segment (start 112.15 105.998) (end 112.226 105.922) (width 0.254) (layer F.Cu) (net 13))
 (segment (start 112.226 105.922) (end 112.226 104.098) (width 0.254) (layer F.Cu) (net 13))
 (segment (start 112.226 104.098) (end 111.445 103.317) (width 0.254) (layer F.Cu) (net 13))
 (segment (start 111.445 103.317) (end 111.395 103.317) (width 0.254) (layer F.Cu) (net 13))
 (segment (start 113.395 104.267) (end 115.871 104.267) (width 0.254) (layer F.Cu) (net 14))
 (segment (start 108.077 107.315) (end 110.088 105.304) (width 0.254) (layer F.Cu) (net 15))
 (segment (start 110.088 105.304) (end 110.088 99.7479) (width 0.254) (layer F.Cu) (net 15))
 (segment (start 110.088 99.7479) (end 111.472 98.364) (width 0.254) (layer F.Cu) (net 15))
 (segment (start 111.472 98.364) (end 111.522 98.364) (width 0.254) (layer F.Cu) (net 15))
 (segment (start 113.522 99.314) (end 115.998 99.314) (width 0.254) (layer F.Cu) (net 16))
 (segment (start 108.077 104.775) (end 109.258 103.594) (width 0.254) (layer F.Cu) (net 17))
 (segment (start 109.258 103.594) (end 109.258 95.752) (width 0.254) (layer F.Cu) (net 17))
 (segment (start 109.258 95.752) (end 111.599 93.411) (width 0.254) (layer F.Cu) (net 17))
 (segment (start 111.599 93.411) (end 111.649 93.411) (width 0.254) (layer F.Cu) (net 17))
 (segment (start 113.649 94.361) (end 115.998 94.361) (width 0.254) (layer F.Cu) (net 18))
 (segment (start 92.837 120.015) (end 97.122 120.015) (width 0.254) (layer F.Cu) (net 19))
 (segment (start 97.122 120.015) (end 97.282 120.175) (width 0.254) (layer F.Cu) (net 19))
 (segment (start 97.282 120.175) (end 98.186 120.175) (width 0.254) (layer F.Cu) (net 19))
 (segment (start 98.186 120.175) (end 100.711 117.65) (width 0.254) (layer F.Cu) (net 19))
 (segment (start 100.711 117.65) (end 100.711 105.791) (width 0.254) (layer F.Cu) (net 19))
 (segment (start 98.171 105.791) (end 98.171 107.442) (width 0.254) (layer F.Cu) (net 21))
 (segment (start 98.171 107.442) (end 98.298 107.569) (width 0.254) (layer F.Cu) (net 21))
 (segment (start 98.298 107.569) (end 106.172 99.695) (width 0.254) (layer B.Cu) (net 21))
 (segment (start 106.172 99.695) (end 108.077 99.695) (width 0.254) (layer B.Cu) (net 21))
 (via (at 98.298 107.569) (size 0.6858) (layers F.Cu B.Cu) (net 21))
 (segment (start 101.981 105.791) (end 101.981 103.251) (width 0.254) (layer F.Cu) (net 22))
 (segment (start 101.981 103.251) (end 108.077 97.155) (width 0.254) (layer F.Cu) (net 22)))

